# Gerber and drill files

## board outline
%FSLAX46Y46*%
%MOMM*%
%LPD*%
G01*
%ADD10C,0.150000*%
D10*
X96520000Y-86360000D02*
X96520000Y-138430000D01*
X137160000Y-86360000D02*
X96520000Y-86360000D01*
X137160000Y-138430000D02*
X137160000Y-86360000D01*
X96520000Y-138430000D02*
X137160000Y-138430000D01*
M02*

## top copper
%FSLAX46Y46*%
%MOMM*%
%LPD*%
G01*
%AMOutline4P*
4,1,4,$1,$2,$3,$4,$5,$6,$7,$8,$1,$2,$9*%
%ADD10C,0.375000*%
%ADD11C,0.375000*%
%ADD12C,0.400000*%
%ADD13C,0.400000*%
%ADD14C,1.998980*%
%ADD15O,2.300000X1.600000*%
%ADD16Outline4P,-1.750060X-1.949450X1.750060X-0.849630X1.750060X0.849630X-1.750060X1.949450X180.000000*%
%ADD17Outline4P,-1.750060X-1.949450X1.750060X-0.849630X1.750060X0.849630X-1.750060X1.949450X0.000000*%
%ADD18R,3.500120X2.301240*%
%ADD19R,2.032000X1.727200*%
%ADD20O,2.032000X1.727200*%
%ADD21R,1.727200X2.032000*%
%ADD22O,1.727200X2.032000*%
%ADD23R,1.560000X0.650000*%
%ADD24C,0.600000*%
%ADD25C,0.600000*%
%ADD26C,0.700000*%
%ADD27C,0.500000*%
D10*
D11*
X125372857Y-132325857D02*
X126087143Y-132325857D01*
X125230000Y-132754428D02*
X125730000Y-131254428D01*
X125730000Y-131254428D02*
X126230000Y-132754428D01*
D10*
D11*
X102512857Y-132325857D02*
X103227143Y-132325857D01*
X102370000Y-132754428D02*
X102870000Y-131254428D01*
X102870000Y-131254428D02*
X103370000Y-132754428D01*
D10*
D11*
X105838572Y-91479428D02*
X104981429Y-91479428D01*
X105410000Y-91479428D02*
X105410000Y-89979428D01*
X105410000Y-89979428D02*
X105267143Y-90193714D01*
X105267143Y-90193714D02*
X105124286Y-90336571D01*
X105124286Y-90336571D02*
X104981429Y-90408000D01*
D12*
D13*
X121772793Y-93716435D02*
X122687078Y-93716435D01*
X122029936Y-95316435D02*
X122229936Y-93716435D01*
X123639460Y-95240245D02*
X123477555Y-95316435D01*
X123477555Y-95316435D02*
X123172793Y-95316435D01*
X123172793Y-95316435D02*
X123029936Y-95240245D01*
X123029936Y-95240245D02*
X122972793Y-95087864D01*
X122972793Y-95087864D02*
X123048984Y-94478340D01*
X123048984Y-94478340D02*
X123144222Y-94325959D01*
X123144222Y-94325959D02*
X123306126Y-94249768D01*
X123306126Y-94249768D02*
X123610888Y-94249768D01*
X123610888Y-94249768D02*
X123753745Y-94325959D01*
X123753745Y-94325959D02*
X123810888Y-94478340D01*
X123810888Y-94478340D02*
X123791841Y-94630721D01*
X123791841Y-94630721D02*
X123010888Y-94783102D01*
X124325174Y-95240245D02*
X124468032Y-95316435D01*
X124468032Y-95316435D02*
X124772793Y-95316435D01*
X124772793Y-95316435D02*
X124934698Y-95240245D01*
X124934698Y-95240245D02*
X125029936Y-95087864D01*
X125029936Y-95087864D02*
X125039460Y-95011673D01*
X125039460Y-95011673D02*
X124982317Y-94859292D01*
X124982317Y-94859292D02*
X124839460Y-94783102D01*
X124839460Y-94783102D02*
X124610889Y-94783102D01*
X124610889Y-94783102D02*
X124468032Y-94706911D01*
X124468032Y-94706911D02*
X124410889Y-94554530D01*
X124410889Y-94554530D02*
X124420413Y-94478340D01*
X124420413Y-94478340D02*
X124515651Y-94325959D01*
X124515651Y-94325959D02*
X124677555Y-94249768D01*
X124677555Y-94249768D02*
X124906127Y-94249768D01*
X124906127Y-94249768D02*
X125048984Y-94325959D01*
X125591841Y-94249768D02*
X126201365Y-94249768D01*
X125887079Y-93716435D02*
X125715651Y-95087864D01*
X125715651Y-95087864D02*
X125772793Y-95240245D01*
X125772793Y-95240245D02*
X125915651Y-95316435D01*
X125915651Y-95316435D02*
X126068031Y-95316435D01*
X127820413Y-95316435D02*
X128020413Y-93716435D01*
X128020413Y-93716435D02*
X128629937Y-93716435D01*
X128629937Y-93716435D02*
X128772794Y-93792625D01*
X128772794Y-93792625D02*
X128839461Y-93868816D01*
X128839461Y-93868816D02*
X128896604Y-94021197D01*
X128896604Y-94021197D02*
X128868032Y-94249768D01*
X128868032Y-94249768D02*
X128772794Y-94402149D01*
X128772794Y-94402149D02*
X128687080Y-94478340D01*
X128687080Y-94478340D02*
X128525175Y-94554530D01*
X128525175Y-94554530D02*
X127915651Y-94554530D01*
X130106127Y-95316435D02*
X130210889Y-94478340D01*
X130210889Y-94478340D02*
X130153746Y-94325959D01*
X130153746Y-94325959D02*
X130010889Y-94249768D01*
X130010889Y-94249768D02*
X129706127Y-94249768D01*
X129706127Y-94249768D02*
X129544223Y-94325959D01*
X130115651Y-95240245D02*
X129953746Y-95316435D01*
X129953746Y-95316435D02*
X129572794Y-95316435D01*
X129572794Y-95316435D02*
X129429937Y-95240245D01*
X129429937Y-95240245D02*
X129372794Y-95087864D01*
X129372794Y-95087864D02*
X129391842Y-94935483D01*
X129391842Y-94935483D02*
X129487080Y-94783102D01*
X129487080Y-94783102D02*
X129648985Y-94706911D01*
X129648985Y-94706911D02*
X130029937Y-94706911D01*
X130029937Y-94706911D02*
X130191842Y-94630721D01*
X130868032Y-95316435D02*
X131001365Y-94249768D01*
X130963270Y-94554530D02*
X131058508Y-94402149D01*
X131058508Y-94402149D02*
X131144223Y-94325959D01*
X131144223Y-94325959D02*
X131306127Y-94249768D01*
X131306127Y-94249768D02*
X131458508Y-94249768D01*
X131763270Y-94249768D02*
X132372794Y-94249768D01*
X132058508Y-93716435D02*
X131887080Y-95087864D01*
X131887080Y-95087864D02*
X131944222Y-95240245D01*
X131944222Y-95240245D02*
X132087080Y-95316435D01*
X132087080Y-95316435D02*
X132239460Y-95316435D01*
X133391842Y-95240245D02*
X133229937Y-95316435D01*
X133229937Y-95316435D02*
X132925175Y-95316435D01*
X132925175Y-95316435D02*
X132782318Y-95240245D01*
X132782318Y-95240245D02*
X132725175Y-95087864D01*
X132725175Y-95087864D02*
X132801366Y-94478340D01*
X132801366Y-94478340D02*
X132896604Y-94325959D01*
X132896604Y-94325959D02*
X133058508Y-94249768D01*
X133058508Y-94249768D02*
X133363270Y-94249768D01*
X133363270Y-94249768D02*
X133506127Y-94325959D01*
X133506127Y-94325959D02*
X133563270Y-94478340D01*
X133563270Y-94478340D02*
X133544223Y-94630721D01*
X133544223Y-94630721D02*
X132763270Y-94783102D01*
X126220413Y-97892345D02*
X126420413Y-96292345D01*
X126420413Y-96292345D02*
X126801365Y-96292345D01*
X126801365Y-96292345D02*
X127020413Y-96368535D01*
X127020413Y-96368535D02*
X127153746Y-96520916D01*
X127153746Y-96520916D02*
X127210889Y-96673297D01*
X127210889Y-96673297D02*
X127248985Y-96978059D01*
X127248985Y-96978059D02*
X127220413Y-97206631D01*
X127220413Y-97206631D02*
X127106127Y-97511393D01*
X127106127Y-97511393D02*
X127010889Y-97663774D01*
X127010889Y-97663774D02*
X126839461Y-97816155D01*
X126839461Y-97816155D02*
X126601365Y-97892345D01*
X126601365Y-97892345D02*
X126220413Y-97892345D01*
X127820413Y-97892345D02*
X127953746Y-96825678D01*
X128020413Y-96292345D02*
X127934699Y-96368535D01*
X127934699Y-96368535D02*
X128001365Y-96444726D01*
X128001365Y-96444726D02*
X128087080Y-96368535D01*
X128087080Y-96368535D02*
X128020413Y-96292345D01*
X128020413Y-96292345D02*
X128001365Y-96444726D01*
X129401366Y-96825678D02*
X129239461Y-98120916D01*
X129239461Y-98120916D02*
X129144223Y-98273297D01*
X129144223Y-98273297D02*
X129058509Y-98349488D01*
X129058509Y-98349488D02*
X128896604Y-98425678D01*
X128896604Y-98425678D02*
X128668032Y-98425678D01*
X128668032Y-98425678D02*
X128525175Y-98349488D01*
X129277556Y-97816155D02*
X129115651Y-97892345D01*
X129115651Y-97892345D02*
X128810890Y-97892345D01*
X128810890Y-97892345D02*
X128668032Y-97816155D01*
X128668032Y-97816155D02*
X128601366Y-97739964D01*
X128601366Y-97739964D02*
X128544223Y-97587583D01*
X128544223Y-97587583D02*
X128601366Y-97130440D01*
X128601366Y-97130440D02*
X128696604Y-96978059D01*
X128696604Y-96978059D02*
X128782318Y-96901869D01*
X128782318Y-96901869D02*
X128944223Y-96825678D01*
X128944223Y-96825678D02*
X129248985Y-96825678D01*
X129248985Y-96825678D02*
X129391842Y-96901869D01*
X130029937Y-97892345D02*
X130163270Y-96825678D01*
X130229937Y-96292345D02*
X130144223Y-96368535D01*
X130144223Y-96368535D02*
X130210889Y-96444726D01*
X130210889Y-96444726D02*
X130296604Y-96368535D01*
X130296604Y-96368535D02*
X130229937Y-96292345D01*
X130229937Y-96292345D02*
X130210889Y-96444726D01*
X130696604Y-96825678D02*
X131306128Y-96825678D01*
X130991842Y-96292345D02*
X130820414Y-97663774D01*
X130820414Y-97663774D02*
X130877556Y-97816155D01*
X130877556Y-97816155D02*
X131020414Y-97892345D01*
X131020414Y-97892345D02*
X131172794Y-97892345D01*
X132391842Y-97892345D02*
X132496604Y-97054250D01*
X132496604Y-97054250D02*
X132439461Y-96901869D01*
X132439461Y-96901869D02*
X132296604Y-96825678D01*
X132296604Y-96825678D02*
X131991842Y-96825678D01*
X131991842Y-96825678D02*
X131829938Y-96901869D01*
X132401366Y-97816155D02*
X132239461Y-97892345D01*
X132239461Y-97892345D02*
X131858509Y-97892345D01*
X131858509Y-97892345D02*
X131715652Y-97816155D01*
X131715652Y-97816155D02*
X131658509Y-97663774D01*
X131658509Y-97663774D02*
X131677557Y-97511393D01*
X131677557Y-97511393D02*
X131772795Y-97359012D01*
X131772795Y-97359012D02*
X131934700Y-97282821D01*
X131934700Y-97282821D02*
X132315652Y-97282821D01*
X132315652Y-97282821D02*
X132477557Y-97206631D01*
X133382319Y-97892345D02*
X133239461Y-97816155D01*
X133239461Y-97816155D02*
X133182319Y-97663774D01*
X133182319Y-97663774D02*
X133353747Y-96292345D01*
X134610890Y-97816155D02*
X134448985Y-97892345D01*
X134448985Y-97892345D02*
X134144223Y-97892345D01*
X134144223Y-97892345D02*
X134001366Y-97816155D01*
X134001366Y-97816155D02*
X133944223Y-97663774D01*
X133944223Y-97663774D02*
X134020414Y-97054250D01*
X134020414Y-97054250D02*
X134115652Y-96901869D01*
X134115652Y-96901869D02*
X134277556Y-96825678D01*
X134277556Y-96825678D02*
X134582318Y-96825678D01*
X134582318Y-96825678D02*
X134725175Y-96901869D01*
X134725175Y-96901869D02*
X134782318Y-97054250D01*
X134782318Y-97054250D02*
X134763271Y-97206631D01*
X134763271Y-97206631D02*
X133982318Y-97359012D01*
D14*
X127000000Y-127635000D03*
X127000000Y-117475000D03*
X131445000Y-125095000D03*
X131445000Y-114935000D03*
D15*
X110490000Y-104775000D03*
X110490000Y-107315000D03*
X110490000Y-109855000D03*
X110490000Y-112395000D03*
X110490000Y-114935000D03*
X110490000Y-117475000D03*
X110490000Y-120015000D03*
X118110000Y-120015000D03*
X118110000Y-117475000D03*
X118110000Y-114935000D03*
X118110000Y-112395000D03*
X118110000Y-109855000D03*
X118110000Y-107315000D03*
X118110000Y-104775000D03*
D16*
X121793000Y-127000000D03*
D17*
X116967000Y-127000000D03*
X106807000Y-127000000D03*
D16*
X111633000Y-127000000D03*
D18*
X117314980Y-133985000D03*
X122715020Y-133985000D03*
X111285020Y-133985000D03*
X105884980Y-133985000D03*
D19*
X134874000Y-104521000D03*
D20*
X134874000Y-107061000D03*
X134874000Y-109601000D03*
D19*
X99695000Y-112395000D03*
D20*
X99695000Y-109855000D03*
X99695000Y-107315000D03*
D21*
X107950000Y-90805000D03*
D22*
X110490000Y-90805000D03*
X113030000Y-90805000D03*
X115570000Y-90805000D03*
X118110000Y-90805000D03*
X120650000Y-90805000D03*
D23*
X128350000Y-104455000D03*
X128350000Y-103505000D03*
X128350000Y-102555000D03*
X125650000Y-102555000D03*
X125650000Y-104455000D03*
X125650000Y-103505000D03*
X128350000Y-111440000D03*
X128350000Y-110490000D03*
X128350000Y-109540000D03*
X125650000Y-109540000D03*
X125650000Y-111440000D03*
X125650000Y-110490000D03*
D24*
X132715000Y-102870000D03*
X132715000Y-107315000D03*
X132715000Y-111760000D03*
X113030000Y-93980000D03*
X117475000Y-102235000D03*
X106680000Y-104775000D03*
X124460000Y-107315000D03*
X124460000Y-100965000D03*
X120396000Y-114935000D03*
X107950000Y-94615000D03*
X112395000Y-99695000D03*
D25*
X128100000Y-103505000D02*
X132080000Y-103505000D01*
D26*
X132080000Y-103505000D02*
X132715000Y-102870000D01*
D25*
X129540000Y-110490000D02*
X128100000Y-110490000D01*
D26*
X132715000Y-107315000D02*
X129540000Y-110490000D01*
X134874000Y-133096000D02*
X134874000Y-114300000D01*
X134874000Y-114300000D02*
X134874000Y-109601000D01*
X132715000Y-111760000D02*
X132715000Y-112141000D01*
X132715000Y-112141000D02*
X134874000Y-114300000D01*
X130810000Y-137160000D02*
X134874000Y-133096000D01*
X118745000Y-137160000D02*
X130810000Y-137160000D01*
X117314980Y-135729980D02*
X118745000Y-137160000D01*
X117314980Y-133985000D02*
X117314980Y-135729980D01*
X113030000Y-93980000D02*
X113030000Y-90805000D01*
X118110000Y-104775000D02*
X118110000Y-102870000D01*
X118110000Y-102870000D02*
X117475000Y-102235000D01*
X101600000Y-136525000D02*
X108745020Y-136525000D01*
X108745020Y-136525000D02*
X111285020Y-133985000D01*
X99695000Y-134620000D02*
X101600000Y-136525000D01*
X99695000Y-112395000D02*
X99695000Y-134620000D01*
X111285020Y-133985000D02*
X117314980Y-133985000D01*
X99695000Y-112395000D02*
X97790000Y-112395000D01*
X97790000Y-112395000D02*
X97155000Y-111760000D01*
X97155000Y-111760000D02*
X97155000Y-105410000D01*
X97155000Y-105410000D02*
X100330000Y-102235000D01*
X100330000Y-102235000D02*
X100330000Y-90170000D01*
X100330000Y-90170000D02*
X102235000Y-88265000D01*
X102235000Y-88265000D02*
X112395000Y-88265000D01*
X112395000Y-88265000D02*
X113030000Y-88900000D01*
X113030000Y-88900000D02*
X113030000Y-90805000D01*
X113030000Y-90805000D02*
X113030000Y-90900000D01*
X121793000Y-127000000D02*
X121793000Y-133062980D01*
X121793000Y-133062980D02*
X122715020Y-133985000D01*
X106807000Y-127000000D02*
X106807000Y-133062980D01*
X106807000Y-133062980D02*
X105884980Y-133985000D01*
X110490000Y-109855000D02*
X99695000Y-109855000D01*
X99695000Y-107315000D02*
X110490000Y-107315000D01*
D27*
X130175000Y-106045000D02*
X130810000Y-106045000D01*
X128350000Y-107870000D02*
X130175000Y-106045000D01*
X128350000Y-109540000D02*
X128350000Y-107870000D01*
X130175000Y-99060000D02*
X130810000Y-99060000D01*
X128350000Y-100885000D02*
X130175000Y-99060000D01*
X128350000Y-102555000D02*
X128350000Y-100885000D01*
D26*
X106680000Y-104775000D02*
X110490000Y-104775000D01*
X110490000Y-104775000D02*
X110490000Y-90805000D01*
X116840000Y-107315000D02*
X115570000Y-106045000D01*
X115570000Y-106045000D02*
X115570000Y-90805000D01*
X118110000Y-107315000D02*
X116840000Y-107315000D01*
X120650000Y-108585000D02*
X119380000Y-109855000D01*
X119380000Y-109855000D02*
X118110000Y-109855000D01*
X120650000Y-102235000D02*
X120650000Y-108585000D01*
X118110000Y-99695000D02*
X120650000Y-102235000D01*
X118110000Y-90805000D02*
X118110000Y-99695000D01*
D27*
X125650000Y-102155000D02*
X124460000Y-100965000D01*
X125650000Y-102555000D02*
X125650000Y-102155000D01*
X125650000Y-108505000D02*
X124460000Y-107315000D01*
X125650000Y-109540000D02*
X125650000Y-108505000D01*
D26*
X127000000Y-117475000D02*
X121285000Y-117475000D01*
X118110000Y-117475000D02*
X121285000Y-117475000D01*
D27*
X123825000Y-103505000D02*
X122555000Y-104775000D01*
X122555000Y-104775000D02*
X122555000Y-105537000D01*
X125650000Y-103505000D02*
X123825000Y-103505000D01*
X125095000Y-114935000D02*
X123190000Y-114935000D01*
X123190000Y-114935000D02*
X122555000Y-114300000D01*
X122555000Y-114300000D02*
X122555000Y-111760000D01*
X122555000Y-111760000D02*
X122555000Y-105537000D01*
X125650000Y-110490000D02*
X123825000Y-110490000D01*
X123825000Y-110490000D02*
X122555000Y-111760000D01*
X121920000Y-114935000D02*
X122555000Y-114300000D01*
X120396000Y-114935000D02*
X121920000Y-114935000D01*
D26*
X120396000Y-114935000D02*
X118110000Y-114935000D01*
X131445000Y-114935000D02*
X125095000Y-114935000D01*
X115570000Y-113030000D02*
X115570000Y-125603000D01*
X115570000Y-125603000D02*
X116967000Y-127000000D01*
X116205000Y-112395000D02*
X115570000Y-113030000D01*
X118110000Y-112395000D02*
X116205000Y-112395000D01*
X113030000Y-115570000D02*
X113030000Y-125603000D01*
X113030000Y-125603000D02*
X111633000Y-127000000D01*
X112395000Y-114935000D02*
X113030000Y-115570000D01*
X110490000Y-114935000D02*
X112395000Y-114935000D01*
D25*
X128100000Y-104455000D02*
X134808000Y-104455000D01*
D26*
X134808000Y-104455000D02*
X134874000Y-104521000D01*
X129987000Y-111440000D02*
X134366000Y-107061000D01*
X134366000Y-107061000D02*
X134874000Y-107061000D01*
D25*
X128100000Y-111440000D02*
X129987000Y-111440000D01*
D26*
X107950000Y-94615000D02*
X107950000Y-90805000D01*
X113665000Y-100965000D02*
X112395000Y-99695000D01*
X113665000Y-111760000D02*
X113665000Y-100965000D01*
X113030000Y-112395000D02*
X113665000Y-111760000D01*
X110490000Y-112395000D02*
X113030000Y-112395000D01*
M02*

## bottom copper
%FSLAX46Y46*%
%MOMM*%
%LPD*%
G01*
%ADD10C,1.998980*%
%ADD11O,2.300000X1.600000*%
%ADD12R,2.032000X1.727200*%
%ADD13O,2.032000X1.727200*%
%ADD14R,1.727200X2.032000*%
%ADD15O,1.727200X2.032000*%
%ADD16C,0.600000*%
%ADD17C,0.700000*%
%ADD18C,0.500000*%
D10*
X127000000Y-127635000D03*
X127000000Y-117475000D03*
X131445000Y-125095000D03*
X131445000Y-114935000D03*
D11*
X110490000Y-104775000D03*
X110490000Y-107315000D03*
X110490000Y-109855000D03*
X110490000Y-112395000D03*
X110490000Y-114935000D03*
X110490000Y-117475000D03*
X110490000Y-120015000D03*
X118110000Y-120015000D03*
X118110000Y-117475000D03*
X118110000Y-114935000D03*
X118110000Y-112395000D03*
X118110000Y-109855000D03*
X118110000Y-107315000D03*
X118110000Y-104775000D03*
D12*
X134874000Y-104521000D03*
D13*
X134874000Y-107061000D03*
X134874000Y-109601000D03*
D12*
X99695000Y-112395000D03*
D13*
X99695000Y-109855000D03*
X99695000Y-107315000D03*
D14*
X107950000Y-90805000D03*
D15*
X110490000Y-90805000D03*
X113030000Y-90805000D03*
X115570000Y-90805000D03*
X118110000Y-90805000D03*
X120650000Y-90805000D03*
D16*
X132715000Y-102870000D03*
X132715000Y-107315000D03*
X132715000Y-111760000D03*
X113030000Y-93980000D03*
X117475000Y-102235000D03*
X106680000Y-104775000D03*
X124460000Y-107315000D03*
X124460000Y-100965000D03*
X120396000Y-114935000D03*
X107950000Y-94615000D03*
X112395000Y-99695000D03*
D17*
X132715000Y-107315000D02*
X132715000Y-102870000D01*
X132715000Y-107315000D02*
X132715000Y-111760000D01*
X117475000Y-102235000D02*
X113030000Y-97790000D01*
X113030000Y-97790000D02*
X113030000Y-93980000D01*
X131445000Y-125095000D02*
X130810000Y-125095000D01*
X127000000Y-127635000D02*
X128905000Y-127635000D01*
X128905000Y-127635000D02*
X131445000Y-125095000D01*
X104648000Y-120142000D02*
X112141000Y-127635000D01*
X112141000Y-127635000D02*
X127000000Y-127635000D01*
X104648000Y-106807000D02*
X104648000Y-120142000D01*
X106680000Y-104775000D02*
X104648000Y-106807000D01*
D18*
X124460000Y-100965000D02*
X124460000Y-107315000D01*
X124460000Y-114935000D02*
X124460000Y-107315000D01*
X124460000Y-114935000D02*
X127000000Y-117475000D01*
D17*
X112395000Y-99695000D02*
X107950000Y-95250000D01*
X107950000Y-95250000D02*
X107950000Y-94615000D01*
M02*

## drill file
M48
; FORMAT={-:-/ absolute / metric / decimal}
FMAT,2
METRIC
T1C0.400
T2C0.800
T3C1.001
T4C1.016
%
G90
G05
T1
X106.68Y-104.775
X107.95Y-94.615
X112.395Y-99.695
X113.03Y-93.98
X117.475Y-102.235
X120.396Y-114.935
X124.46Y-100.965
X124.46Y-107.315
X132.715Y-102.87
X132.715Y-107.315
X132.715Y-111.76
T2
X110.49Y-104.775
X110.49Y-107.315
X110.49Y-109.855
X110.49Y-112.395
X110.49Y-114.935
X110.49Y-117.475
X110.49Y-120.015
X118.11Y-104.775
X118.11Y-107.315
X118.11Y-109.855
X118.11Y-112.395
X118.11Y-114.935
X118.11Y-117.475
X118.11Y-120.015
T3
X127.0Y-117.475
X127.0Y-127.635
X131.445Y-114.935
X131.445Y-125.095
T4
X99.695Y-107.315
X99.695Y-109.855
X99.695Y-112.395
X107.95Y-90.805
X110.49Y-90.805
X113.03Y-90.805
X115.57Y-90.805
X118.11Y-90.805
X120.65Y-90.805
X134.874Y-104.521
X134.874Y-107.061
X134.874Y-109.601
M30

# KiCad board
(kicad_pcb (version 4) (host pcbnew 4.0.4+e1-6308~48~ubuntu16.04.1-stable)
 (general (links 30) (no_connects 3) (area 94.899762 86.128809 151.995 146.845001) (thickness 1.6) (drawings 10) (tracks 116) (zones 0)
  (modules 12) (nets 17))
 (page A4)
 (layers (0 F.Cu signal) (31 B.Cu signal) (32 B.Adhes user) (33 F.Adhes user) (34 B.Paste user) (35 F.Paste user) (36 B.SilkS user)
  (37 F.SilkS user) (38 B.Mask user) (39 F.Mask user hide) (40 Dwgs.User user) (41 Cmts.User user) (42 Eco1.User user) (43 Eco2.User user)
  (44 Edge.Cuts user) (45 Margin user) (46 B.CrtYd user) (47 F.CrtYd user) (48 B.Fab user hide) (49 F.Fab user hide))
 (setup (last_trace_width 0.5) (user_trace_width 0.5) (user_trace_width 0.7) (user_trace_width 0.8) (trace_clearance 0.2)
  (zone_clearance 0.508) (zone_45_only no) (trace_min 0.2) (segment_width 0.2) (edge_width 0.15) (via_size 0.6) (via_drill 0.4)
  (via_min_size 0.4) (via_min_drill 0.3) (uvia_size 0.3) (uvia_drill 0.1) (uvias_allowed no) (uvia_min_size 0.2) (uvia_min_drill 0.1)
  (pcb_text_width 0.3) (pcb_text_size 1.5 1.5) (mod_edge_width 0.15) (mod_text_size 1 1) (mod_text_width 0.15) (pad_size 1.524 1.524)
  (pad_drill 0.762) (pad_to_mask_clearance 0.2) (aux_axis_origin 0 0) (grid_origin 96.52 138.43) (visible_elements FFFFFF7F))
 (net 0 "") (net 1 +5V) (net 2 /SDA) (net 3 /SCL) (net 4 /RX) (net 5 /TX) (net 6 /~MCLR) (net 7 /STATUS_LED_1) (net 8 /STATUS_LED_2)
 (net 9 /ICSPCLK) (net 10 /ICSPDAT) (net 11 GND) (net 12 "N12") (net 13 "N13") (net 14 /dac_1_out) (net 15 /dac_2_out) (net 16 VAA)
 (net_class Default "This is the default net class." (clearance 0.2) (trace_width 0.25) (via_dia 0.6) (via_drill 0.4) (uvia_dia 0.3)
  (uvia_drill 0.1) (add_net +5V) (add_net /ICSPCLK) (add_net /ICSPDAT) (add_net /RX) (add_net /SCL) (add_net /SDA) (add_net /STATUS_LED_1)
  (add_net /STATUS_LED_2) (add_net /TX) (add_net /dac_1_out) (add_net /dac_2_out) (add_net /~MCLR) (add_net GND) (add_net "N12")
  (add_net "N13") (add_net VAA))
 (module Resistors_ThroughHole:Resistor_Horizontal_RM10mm (layer F.Cu) (at 127 127.635 90)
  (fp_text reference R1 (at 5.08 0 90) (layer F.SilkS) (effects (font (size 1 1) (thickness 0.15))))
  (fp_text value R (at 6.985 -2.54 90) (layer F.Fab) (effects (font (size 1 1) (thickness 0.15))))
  (pad 1 thru_hole circle (at 0 0 90) (size 1.99898 1.99898) (drill 1.00076) (layers *.Cu *.SilkS *.Mask) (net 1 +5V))
  (pad 2 thru_hole circle (at 10.16 0 90) (size 1.99898 1.99898) (drill 1.00076) (layers *.Cu *.SilkS *.Mask) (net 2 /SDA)))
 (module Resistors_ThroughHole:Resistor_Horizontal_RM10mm (layer F.Cu) (at 131.445 125.095 90)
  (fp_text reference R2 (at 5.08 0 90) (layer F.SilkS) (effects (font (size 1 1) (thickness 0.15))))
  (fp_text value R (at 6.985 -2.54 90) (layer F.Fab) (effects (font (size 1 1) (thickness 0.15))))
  (pad 1 thru_hole circle (at 0 0 90) (size 1.99898 1.99898) (drill 1.00076) (layers *.Cu *.SilkS *.Mask) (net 1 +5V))
  (pad 2 thru_hole circle (at 10.16 0 90) (size 1.99898 1.99898) (drill 1.00076) (layers *.Cu *.SilkS *.Mask) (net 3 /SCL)))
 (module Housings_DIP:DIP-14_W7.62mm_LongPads (layer F.Cu) (at 110.49 104.775)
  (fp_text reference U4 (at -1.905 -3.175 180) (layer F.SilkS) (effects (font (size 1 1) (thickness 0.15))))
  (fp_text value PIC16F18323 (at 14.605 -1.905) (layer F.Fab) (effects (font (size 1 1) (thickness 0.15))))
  (pad 1 thru_hole oval (at 0 0) (size 2.3 1.6) (drill 0.8) (layers *.Cu *.Mask F.SilkS) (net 1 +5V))
  (pad 2 thru_hole oval (at 0 2.54) (size 2.3 1.6) (drill 0.8) (layers *.Cu *.Mask F.SilkS) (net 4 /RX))
  (pad 3 thru_hole oval (at 0 5.08) (size 2.3 1.6) (drill 0.8) (layers *.Cu *.Mask F.SilkS) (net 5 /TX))
  (pad 4 thru_hole oval (at 0 7.62) (size 2.3 1.6) (drill 0.8) (layers *.Cu *.Mask F.SilkS) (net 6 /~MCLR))
  (pad 5 thru_hole oval (at 0 10.16) (size 2.3 1.6) (drill 0.8) (layers *.Cu *.Mask F.SilkS) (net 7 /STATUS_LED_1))
  (pad 6 thru_hole oval (at 0 12.7) (size 2.3 1.6) (drill 0.8) (layers *.Cu *.Mask F.SilkS))
  (pad 7 thru_hole oval (at 0 15.24) (size 2.3 1.6) (drill 0.8) (layers *.Cu *.Mask F.SilkS))
  (pad 8 thru_hole oval (at 7.62 15.24) (size 2.3 1.6) (drill 0.8) (layers *.Cu *.Mask F.SilkS))
  (pad 9 thru_hole oval (at 7.62 12.7) (size 2.3 1.6) (drill 0.8) (layers *.Cu *.Mask F.SilkS) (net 2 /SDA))
  (pad 10 thru_hole oval (at 7.62 10.16) (size 2.3 1.6) (drill 0.8) (layers *.Cu *.Mask F.SilkS) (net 3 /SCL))
  (pad 11 thru_hole oval (at 7.62 7.62) (size 2.3 1.6) (drill 0.8) (layers *.Cu *.Mask F.SilkS) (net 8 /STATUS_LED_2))
  (pad 12 thru_hole oval (at 7.62 5.08) (size 2.3 1.6) (drill 0.8) (layers *.Cu *.Mask F.SilkS) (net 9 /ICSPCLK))
  (pad 13 thru_hole oval (at 7.62 2.54) (size 2.3 1.6) (drill 0.8) (layers *.Cu *.Mask F.SilkS) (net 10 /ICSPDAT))
  (pad 14 thru_hole oval (at 7.62 0) (size 2.3 1.6) (drill 0.8) (layers *.Cu *.Mask F.SilkS) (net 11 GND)))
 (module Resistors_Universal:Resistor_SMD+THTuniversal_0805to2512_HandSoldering (layer F.Cu) (at 119.38 127 180)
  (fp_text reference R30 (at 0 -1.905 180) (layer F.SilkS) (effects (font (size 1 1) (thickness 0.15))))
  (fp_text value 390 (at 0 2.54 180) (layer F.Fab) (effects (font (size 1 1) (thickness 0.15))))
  (pad 1 smd trapezoid (at -2.413 0 180) (size 3.50012 2.79908) (rect_delta 1.09982 0) (layers F.Cu F.Paste F.Mask) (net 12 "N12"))
  (pad 2 smd trapezoid (at 2.413 0) (size 3.50012 2.79908) (rect_delta 1.09982 0) (layers F.Cu F.Paste F.Mask) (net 8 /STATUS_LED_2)))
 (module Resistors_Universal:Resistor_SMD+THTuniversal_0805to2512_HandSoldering (layer F.Cu) (at 109.22 127)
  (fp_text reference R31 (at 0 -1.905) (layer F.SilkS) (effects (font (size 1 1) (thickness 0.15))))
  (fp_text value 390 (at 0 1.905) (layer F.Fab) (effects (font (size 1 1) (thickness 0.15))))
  (pad 1 smd trapezoid (at -2.413 0) (size 3.50012 2.79908) (rect_delta 1.09982 0) (layers F.Cu F.Paste F.Mask) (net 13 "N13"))
  (pad 2 smd trapezoid (at 2.413 0 180) (size 3.50012 2.79908) (rect_delta 1.09982 0) (layers F.Cu F.Paste F.Mask) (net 7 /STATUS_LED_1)))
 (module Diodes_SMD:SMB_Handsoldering (layer F.Cu) (at 120.015 133.985)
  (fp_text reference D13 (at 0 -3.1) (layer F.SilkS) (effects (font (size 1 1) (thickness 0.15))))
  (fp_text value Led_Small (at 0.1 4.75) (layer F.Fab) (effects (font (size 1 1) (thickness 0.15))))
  (pad 1 smd rect (at -2.70002 0) (size 3.50012 2.30124) (layers F.Cu F.Paste F.Mask) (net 11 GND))
  (pad 2 smd rect (at 2.70002 0) (size 3.50012 2.30124) (layers F.Cu F.Paste F.Mask) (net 12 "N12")))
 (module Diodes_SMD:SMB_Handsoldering (layer F.Cu) (at 108.585 133.985 180)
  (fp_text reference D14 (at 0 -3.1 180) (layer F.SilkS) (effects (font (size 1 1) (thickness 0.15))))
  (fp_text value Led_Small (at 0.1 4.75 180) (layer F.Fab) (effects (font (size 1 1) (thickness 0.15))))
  (pad 1 smd rect (at -2.70002 0 180) (size 3.50012 2.30124) (layers F.Cu F.Paste F.Mask) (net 11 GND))
  (pad 2 smd rect (at 2.70002 0 180) (size 3.50012 2.30124) (layers F.Cu F.Paste F.Mask) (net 13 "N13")))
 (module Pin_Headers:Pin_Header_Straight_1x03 (layer F.Cu) (at 134.874 104.521)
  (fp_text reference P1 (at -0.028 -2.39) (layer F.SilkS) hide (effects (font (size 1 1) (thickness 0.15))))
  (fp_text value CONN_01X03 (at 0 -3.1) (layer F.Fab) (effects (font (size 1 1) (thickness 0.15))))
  (pad 1 thru_hole rect (at 0 0) (size 2.032 1.7272) (drill 1.016) (layers *.Cu *.Mask F.SilkS) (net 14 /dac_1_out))
  (pad 2 thru_hole oval (at 0 2.54) (size 2.032 1.7272) (drill 1.016) (layers *.Cu *.Mask F.SilkS) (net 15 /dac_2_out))
  (pad 3 thru_hole oval (at 0 5.08) (size 2.032 1.7272) (drill 1.016) (layers *.Cu *.Mask F.SilkS) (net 11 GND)))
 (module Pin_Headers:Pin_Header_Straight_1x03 (layer F.Cu) (at 99.695 112.395 180)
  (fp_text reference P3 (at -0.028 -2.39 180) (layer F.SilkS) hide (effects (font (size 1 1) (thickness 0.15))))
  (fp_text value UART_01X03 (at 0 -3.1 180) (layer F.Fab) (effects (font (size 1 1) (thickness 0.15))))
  (pad 1 thru_hole rect (at 0 0 180) (size 2.032 1.7272) (drill 1.016) (layers *.Cu *.Mask F.SilkS) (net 11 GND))
  (pad 2 thru_hole oval (at 0 2.54 180) (size 2.032 1.7272) (drill 1.016) (layers *.Cu *.Mask F.SilkS) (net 5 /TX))
  (pad 3 thru_hole oval (at 0 5.08 180) (size 2.032 1.7272) (drill 1.016) (layers *.Cu *.Mask F.SilkS) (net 4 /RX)))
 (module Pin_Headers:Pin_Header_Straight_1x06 (layer F.Cu) (at 107.95 90.805 90)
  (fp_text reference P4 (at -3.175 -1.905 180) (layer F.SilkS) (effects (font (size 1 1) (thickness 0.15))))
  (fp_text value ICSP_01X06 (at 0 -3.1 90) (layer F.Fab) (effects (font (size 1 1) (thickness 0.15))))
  (pad 1 thru_hole rect (at 0 0 90) (size 2.032 1.7272) (drill 1.016) (layers *.Cu *.Mask F.SilkS) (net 6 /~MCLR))
  (pad 2 thru_hole oval (at 0 2.54 90) (size 2.032 1.7272) (drill 1.016) (layers *.Cu *.Mask F.SilkS) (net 1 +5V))
  (pad 3 thru_hole oval (at 0 5.08 90) (size 2.032 1.7272) (drill 1.016) (layers *.Cu *.Mask F.SilkS) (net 11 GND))
  (pad 4 thru_hole oval (at 0 7.62 90) (size 2.032 1.7272) (drill 1.016) (layers *.Cu *.Mask F.SilkS) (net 10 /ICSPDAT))
  (pad 5 thru_hole oval (at 0 10.16 90) (size 2.032 1.7272) (drill 1.016) (layers *.Cu *.Mask F.SilkS) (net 9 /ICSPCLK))
  (pad 6 thru_hole oval (at 0 12.7 90) (size 2.032 1.7272) (drill 1.016) (layers *.Cu *.Mask F.SilkS)))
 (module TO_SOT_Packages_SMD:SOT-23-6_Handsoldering (layer F.Cu) (at 127 103.505 180)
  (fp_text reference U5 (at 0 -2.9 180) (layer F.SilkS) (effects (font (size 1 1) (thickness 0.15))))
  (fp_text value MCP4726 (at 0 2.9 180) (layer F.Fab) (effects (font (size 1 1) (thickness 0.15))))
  (pad 1 smd rect (at -1.35 -0.95 180) (size 1.56 0.65) (layers F.Cu F.Paste F.Mask) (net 14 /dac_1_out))
  (pad 2 smd rect (at -1.35 0 180) (size 1.56 0.65) (layers F.Cu F.Paste F.Mask) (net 11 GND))
  (pad 3 smd rect (at -1.35 0.95 180) (size 1.56 0.65) (layers F.Cu F.Paste F.Mask) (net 1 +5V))
  (pad 4 smd rect (at 1.35 0.95 180) (size 1.56 0.65) (layers F.Cu F.Paste F.Mask) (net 2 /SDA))
  (pad 6 smd rect (at 1.35 -0.95 180) (size 1.56 0.65) (layers F.Cu F.Paste F.Mask) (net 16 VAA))
  (pad 5 smd rect (at 1.35 0 180) (size 1.56 0.65) (layers F.Cu F.Paste F.Mask) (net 3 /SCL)))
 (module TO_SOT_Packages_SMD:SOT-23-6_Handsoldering (layer F.Cu) (at 127 110.49 180)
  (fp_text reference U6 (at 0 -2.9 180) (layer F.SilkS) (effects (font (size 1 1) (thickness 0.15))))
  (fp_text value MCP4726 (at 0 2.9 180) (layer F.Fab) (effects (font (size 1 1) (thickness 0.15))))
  (pad 1 smd rect (at -1.35 -0.95 180) (size 1.56 0.65) (layers F.Cu F.Paste F.Mask) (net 15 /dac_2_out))
  (pad 2 smd rect (at -1.35 0 180) (size 1.56 0.65) (layers F.Cu F.Paste F.Mask) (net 11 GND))
  (pad 3 smd rect (at -1.35 0.95 180) (size 1.56 0.65) (layers F.Cu F.Paste F.Mask) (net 1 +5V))
  (pad 4 smd rect (at 1.35 0.95 180) (size 1.56 0.65) (layers F.Cu F.Paste F.Mask) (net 2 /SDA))
  (pad 6 smd rect (at 1.35 -0.95 180) (size 1.56 0.65) (layers F.Cu F.Paste F.Mask) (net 16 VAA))
  (pad 5 smd rect (at 1.35 0 180) (size 1.56 0.65) (layers F.Cu F.Paste F.Mask) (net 3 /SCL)))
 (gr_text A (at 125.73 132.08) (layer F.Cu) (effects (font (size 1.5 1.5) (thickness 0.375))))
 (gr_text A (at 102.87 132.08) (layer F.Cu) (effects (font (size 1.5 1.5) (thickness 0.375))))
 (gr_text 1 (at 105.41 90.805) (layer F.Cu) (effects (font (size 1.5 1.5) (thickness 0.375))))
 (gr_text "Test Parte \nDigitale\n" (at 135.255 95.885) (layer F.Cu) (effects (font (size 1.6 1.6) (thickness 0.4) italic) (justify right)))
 (gr_line (start 96.52 86.36) (end 96.52 138.43) (angle 90) (layer Edge.Cuts) (width 0.15))
 (gr_line (start 137.16 86.36) (end 96.52 86.36) (angle 90) (layer Edge.Cuts) (width 0.15))
 (gr_line (start 137.16 138.43) (end 137.16 86.36) (angle 90) (layer Edge.Cuts) (width 0.15))
 (gr_line (start 96.52 138.43) (end 137.16 138.43) (angle 90) (layer Edge.Cuts) (width 0.15))
 (segment (start 128.1 103.505) (end 132.08 103.505) (width 0.6) (layer F.Cu) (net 11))
 (segment (start 132.08 103.505) (end 132.715 102.87) (width 0.7) (layer F.Cu) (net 11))
 (via (at 132.715 102.87) (size 0.6) (drill 0.4) (layers F.Cu B.Cu) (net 11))
 (segment (start 132.715 107.315) (end 132.715 102.87) (width 0.7) (layer B.Cu) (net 11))
 (via (at 132.715 107.315) (size 0.6) (drill 0.4) (layers F.Cu B.Cu) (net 11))
 (segment (start 129.54 110.49) (end 128.1 110.49) (width 0.6) (layer F.Cu) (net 11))
 (segment (start 132.715 107.315) (end 129.54 110.49) (width 0.7) (layer F.Cu) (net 11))
 (segment (start 132.715 107.315) (end 132.715 111.76) (width 0.7) (layer B.Cu) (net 11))
 (segment (start 134.874 133.096) (end 134.874 114.3) (width 0.7) (layer F.Cu) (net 11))
 (segment (start 134.874 114.3) (end 134.874 109.601) (width 0.7) (layer F.Cu) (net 11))
 (segment (start 132.715 111.76) (end 132.715 112.141) (width 0.7) (layer F.Cu) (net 11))
 (segment (start 132.715 112.141) (end 134.874 114.3) (width 0.7) (layer F.Cu) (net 11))
 (via (at 132.715 111.76) (size 0.6) (drill 0.4) (layers F.Cu B.Cu) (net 11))
 (segment (start 130.81 137.16) (end 134.874 133.096) (width 0.7) (layer F.Cu) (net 11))
 (segment (start 118.745 137.16) (end 130.81 137.16) (width 0.7) (layer F.Cu) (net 11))
 (segment (start 117.31498 135.72998) (end 118.745 137.16) (width 0.7) (layer F.Cu) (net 11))
 (segment (start 117.31498 133.985) (end 117.31498 135.72998) (width 0.7) (layer F.Cu) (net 11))
 (segment (start 113.03 93.98) (end 113.03 90.805) (width 0.7) (layer F.Cu) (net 11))
 (segment (start 117.475 102.235) (end 113.03 97.79) (width 0.7) (layer B.Cu) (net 11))
 (segment (start 113.03 97.79) (end 113.03 93.98) (width 0.7) (layer B.Cu) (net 11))
 (via (at 113.03 93.98) (size 0.6) (drill 0.4) (layers F.Cu B.Cu) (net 11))
 (segment (start 118.11 104.775) (end 118.11 102.87) (width 0.7) (layer F.Cu) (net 11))
 (segment (start 118.11 102.87) (end 117.475 102.235) (width 0.7) (layer F.Cu) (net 11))
 (via (at 117.475 102.235) (size 0.6) (drill 0.4) (layers F.Cu B.Cu) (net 11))
 (segment (start 101.6 136.525) (end 108.74502 136.525) (width 0.7) (layer F.Cu) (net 11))
 (segment (start 108.74502 136.525) (end 111.28502 133.985) (width 0.7) (layer F.Cu) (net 11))
 (segment (start 99.695 134.62) (end 101.6 136.525) (width 0.7) (layer F.Cu) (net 11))
 (segment (start 99.695 112.395) (end 99.695 134.62) (width 0.7) (layer F.Cu) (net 11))
 (segment (start 111.28502 133.985) (end 117.31498 133.985) (width 0.7) (layer F.Cu) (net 11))
 (segment (start 99.695 112.395) (end 97.79 112.395) (width 0.7) (layer F.Cu) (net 11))
 (segment (start 97.79 112.395) (end 97.155 111.76) (width 0.7) (layer F.Cu) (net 11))
 (segment (start 97.155 111.76) (end 97.155 105.41) (width 0.7) (layer F.Cu) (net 11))
 (segment (start 97.155 105.41) (end 100.33 102.235) (width 0.7) (layer F.Cu) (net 11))
 (segment (start 100.33 102.235) (end 100.33 90.17) (width 0.7) (layer F.Cu) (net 11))
 (segment (start 100.33 90.17) (end 102.235 88.265) (width 0.7) (layer F.Cu) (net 11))
 (segment (start 102.235 88.265) (end 112.395 88.265) (width 0.7) (layer F.Cu) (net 11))
 (segment (start 112.395 88.265) (end 113.03 88.9) (width 0.7) (layer F.Cu) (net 11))
 (segment (start 113.03 88.9) (end 113.03 90.805) (width 0.7) (layer F.Cu) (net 11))
 (segment (start 113.03 90.805) (end 113.03 90.9) (width 0.7) (layer F.Cu) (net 11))
 (segment (start 121.793 127) (end 121.793 133.06298) (width 0.7) (layer F.Cu) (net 12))
 (segment (start 121.793 133.06298) (end 122.71502 133.985) (width 0.7) (layer F.Cu) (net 12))
 (segment (start 106.807 127) (end 106.807 133.06298) (width 0.7) (layer F.Cu) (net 13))
 (segment (start 106.807 133.06298) (end 105.88498 133.985) (width 0.7) (layer F.Cu) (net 13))
 (segment (start 110.49 109.855) (end 99.695 109.855) (width 0.7) (layer F.Cu) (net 5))
 (segment (start 99.695 107.315) (end 110.49 107.315) (width 0.7) (layer F.Cu) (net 4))
 (segment (start 130.175 106.045) (end 130.81 106.045) (width 0.5) (layer F.Cu) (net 1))
 (segment (start 128.35 107.87) (end 130.175 106.045) (width 0.5) (layer F.Cu) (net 1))
 (segment (start 128.35 109.54) (end 128.35 107.87) (width 0.5) (layer F.Cu) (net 1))
 (segment (start 130.175 99.06) (end 130.81 99.06) (width 0.5) (layer F.Cu) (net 1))
 (segment (start 128.35 100.885) (end 130.175 99.06) (width 0.5) (layer F.Cu) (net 1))
 (segment (start 128.35 102.555) (end 128.35 100.885) (width 0.5) (layer F.Cu) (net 1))
 (segment (start 106.68 104.775) (end 110.49 104.775) (width 0.7) (layer F.Cu) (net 1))
 (via (at 106.68 104.775) (size 0.6) (drill 0.4) (layers F.Cu B.Cu) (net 1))
 (segment (start 131.445 125.095) (end 130.81 125.095) (width 0.7) (layer B.Cu) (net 1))
 (segment (start 127 127.635) (end 128.905 127.635) (width 0.7) (layer B.Cu) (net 1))
 (segment (start 128.905 127.635) (end 131.445 125.095) (width 0.7) (layer B.Cu) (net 1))
 (segment (start 104.648 120.142) (end 112.141 127.635) (width 0.7) (layer B.Cu) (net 1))
 (segment (start 112.141 127.635) (end 127 127.635) (width 0.7) (layer B.Cu) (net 1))
 (segment (start 104.648 106.807) (end 104.648 120.142) (width 0.7) (layer B.Cu) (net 1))
 (segment (start 106.68 104.775) (end 104.648 106.807) (width 0.7) (layer B.Cu) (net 1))
 (segment (start 110.49 104.775) (end 110.49 90.805) (width 0.7) (layer F.Cu) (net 1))
 (segment (start 116.84 107.315) (end 115.57 106.045) (width 0.7) (layer F.Cu) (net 10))
 (segment (start 115.57 106.045) (end 115.57 90.805) (width 0.7) (layer F.Cu) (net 10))
 (segment (start 118.11 107.315) (end 116.84 107.315) (width 0.7) (layer F.Cu) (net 10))
 (segment (start 120.65 108.585) (end 119.38 109.855) (width 0.7) (layer F.Cu) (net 9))
 (segment (start 119.38 109.855) (end 118.11 109.855) (width 0.7) (layer F.Cu) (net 9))
 (segment (start 120.65 102.235) (end 120.65 108.585) (width 0.7) (layer F.Cu) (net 9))
 (segment (start 118.11 99.695) (end 120.65 102.235) (width 0.7) (layer F.Cu) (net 9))
 (segment (start 118.11 90.805) (end 118.11 99.695) (width 0.7) (layer F.Cu) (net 9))
 (segment (start 124.46 100.965) (end 124.46 107.315) (width 0.5) (layer B.Cu) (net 2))
 (segment (start 124.46 114.935) (end 124.46 107.315) (width 0.5) (layer B.Cu) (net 2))
 (via (at 124.46 107.315) (size 0.6) (drill 0.4) (layers F.Cu B.Cu) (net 2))
 (segment (start 124.46 114.935) (end 127 117.475) (width 0.5) (layer B.Cu) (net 2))
 (via (at 124.46 100.965) (size 0.6) (drill 0.4) (layers F.Cu B.Cu) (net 2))
 (segment (start 125.65 102.155) (end 124.46 100.965) (width 0.5) (layer F.Cu) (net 2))
 (segment (start 125.65 102.555) (end 125.65 102.155) (width 0.5) (layer F.Cu) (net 2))
 (segment (start 125.65 108.505) (end 124.46 107.315) (width 0.5) (layer F.Cu) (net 2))
 (segment (start 125.65 109.54) (end 125.65 108.505) (width 0.5) (layer F.Cu) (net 2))
 (segment (start 127 117.475) (end 121.285 117.475) (width 0.7) (layer F.Cu) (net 2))
 (segment (start 118.11 117.475) (end 121.285 117.475) (width 0.7) (layer F.Cu) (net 2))
 (segment (start 123.825 103.505) (end 122.555 104.775) (width 0.5) (layer F.Cu) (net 3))
 (segment (start 122.555 104.775) (end 122.555 105.537) (width 0.5) (layer F.Cu) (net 3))
 (segment (start 125.65 103.505) (end 123.825 103.505) (width 0.5) (layer F.Cu) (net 3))
 (segment (start 125.095 114.935) (end 123.19 114.935) (width 0.5) (layer F.Cu) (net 3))
 (segment (start 123.19 114.935) (end 122.555 114.3) (width 0.5) (layer F.Cu) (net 3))
 (segment (start 122.555 114.3) (end 122.555 111.76) (width 0.5) (layer F.Cu) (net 3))
 (segment (start 122.555 111.76) (end 122.555 105.537) (width 0.5) (layer F.Cu) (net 3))
 (segment (start 125.65 110.49) (end 123.825 110.49) (width 0.5) (layer F.Cu) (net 3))
 (segment (start 123.825 110.49) (end 122.555 111.76) (width 0.5) (layer F.Cu) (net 3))
 (segment (start 121.92 114.935) (end 122.555 114.3) (width 0.5) (layer F.Cu) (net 3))
 (segment (start 120.396 114.935) (end 121.92 114.935) (width 0.5) (layer F.Cu) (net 3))
 (segment (start 120.396 114.935) (end 118.11 114.935) (width 0.7) (layer F.Cu) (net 3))
 (via (at 120.396 114.935) (size 0.6) (drill 0.4) (layers F.Cu B.Cu) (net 3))
 (segment (start 131.445 114.935) (end 125.095 114.935) (width 0.7) (layer F.Cu) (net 3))
 (segment (start 115.57 113.03) (end 115.57 125.603) (width 0.7) (layer F.Cu) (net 8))
 (segment (start 115.57 125.603) (end 116.967 127) (width 0.7) (layer F.Cu) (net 8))
 (segment (start 116.205 112.395) (end 115.57 113.03) (width 0.7) (layer F.Cu) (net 8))
 (segment (start 118.11 112.395) (end 116.205 112.395) (width 0.7) (layer F.Cu) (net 8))
 (segment (start 113.03 115.57) (end 113.03 125.603) (width 0.7) (layer F.Cu) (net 7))
 (segment (start 113.03 125.603) (end 111.633 127) (width 0.7) (layer F.Cu) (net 7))
 (segment (start 112.395 114.935) (end 113.03 115.57) (width 0.7) (layer F.Cu) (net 7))
 (segment (start 110.49 114.935) (end 112.395 114.935) (width 0.7) (layer F.Cu) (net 7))
 (segment (start 128.1 104.455) (end 134.808 104.455) (width 0.6) (layer F.Cu) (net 14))
 (segment (start 134.808 104.455) (end 134.874 104.521) (width 0.7) (layer F.Cu) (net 14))
 (segment (start 129.987 111.44) (end 134.366 107.061) (width 0.7) (layer F.Cu) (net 15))
 (segment (start 134.366 107.061) (end 134.874 107.061) (width 0.7) (layer F.Cu) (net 15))
 (segment (start 128.1 111.44) (end 129.987 111.44) (width 0.6) (layer F.Cu) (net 15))
 (segment (start 107.95 94.615) (end 107.95 90.805) (width 0.7) (layer F.Cu) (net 6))
 (segment (start 112.395 99.695) (end 107.95 95.25) (width 0.7) (layer B.Cu) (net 6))
 (segment (start 107.95 95.25) (end 107.95 94.615) (width 0.7) (layer B.Cu) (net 6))
 (via (at 107.95 94.615) (size 0.6) (drill 0.4) (layers F.Cu B.Cu) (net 6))
 (segment (start 113.665 100.965) (end 112.395 99.695) (width 0.7) (layer F.Cu) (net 6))
 (via (at 112.395 99.695) (size 0.6) (drill 0.4) (layers F.Cu B.Cu) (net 6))
 (segment (start 113.665 111.76) (end 113.665 100.965) (width 0.7) (layer F.Cu) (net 6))
 (segment (start 113.03 112.395) (end 113.665 111.76) (width 0.7) (layer F.Cu) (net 6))
 (segment (start 110.49 112.395) (end 113.03 112.395) (width 0.7) (layer F.Cu) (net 6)))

